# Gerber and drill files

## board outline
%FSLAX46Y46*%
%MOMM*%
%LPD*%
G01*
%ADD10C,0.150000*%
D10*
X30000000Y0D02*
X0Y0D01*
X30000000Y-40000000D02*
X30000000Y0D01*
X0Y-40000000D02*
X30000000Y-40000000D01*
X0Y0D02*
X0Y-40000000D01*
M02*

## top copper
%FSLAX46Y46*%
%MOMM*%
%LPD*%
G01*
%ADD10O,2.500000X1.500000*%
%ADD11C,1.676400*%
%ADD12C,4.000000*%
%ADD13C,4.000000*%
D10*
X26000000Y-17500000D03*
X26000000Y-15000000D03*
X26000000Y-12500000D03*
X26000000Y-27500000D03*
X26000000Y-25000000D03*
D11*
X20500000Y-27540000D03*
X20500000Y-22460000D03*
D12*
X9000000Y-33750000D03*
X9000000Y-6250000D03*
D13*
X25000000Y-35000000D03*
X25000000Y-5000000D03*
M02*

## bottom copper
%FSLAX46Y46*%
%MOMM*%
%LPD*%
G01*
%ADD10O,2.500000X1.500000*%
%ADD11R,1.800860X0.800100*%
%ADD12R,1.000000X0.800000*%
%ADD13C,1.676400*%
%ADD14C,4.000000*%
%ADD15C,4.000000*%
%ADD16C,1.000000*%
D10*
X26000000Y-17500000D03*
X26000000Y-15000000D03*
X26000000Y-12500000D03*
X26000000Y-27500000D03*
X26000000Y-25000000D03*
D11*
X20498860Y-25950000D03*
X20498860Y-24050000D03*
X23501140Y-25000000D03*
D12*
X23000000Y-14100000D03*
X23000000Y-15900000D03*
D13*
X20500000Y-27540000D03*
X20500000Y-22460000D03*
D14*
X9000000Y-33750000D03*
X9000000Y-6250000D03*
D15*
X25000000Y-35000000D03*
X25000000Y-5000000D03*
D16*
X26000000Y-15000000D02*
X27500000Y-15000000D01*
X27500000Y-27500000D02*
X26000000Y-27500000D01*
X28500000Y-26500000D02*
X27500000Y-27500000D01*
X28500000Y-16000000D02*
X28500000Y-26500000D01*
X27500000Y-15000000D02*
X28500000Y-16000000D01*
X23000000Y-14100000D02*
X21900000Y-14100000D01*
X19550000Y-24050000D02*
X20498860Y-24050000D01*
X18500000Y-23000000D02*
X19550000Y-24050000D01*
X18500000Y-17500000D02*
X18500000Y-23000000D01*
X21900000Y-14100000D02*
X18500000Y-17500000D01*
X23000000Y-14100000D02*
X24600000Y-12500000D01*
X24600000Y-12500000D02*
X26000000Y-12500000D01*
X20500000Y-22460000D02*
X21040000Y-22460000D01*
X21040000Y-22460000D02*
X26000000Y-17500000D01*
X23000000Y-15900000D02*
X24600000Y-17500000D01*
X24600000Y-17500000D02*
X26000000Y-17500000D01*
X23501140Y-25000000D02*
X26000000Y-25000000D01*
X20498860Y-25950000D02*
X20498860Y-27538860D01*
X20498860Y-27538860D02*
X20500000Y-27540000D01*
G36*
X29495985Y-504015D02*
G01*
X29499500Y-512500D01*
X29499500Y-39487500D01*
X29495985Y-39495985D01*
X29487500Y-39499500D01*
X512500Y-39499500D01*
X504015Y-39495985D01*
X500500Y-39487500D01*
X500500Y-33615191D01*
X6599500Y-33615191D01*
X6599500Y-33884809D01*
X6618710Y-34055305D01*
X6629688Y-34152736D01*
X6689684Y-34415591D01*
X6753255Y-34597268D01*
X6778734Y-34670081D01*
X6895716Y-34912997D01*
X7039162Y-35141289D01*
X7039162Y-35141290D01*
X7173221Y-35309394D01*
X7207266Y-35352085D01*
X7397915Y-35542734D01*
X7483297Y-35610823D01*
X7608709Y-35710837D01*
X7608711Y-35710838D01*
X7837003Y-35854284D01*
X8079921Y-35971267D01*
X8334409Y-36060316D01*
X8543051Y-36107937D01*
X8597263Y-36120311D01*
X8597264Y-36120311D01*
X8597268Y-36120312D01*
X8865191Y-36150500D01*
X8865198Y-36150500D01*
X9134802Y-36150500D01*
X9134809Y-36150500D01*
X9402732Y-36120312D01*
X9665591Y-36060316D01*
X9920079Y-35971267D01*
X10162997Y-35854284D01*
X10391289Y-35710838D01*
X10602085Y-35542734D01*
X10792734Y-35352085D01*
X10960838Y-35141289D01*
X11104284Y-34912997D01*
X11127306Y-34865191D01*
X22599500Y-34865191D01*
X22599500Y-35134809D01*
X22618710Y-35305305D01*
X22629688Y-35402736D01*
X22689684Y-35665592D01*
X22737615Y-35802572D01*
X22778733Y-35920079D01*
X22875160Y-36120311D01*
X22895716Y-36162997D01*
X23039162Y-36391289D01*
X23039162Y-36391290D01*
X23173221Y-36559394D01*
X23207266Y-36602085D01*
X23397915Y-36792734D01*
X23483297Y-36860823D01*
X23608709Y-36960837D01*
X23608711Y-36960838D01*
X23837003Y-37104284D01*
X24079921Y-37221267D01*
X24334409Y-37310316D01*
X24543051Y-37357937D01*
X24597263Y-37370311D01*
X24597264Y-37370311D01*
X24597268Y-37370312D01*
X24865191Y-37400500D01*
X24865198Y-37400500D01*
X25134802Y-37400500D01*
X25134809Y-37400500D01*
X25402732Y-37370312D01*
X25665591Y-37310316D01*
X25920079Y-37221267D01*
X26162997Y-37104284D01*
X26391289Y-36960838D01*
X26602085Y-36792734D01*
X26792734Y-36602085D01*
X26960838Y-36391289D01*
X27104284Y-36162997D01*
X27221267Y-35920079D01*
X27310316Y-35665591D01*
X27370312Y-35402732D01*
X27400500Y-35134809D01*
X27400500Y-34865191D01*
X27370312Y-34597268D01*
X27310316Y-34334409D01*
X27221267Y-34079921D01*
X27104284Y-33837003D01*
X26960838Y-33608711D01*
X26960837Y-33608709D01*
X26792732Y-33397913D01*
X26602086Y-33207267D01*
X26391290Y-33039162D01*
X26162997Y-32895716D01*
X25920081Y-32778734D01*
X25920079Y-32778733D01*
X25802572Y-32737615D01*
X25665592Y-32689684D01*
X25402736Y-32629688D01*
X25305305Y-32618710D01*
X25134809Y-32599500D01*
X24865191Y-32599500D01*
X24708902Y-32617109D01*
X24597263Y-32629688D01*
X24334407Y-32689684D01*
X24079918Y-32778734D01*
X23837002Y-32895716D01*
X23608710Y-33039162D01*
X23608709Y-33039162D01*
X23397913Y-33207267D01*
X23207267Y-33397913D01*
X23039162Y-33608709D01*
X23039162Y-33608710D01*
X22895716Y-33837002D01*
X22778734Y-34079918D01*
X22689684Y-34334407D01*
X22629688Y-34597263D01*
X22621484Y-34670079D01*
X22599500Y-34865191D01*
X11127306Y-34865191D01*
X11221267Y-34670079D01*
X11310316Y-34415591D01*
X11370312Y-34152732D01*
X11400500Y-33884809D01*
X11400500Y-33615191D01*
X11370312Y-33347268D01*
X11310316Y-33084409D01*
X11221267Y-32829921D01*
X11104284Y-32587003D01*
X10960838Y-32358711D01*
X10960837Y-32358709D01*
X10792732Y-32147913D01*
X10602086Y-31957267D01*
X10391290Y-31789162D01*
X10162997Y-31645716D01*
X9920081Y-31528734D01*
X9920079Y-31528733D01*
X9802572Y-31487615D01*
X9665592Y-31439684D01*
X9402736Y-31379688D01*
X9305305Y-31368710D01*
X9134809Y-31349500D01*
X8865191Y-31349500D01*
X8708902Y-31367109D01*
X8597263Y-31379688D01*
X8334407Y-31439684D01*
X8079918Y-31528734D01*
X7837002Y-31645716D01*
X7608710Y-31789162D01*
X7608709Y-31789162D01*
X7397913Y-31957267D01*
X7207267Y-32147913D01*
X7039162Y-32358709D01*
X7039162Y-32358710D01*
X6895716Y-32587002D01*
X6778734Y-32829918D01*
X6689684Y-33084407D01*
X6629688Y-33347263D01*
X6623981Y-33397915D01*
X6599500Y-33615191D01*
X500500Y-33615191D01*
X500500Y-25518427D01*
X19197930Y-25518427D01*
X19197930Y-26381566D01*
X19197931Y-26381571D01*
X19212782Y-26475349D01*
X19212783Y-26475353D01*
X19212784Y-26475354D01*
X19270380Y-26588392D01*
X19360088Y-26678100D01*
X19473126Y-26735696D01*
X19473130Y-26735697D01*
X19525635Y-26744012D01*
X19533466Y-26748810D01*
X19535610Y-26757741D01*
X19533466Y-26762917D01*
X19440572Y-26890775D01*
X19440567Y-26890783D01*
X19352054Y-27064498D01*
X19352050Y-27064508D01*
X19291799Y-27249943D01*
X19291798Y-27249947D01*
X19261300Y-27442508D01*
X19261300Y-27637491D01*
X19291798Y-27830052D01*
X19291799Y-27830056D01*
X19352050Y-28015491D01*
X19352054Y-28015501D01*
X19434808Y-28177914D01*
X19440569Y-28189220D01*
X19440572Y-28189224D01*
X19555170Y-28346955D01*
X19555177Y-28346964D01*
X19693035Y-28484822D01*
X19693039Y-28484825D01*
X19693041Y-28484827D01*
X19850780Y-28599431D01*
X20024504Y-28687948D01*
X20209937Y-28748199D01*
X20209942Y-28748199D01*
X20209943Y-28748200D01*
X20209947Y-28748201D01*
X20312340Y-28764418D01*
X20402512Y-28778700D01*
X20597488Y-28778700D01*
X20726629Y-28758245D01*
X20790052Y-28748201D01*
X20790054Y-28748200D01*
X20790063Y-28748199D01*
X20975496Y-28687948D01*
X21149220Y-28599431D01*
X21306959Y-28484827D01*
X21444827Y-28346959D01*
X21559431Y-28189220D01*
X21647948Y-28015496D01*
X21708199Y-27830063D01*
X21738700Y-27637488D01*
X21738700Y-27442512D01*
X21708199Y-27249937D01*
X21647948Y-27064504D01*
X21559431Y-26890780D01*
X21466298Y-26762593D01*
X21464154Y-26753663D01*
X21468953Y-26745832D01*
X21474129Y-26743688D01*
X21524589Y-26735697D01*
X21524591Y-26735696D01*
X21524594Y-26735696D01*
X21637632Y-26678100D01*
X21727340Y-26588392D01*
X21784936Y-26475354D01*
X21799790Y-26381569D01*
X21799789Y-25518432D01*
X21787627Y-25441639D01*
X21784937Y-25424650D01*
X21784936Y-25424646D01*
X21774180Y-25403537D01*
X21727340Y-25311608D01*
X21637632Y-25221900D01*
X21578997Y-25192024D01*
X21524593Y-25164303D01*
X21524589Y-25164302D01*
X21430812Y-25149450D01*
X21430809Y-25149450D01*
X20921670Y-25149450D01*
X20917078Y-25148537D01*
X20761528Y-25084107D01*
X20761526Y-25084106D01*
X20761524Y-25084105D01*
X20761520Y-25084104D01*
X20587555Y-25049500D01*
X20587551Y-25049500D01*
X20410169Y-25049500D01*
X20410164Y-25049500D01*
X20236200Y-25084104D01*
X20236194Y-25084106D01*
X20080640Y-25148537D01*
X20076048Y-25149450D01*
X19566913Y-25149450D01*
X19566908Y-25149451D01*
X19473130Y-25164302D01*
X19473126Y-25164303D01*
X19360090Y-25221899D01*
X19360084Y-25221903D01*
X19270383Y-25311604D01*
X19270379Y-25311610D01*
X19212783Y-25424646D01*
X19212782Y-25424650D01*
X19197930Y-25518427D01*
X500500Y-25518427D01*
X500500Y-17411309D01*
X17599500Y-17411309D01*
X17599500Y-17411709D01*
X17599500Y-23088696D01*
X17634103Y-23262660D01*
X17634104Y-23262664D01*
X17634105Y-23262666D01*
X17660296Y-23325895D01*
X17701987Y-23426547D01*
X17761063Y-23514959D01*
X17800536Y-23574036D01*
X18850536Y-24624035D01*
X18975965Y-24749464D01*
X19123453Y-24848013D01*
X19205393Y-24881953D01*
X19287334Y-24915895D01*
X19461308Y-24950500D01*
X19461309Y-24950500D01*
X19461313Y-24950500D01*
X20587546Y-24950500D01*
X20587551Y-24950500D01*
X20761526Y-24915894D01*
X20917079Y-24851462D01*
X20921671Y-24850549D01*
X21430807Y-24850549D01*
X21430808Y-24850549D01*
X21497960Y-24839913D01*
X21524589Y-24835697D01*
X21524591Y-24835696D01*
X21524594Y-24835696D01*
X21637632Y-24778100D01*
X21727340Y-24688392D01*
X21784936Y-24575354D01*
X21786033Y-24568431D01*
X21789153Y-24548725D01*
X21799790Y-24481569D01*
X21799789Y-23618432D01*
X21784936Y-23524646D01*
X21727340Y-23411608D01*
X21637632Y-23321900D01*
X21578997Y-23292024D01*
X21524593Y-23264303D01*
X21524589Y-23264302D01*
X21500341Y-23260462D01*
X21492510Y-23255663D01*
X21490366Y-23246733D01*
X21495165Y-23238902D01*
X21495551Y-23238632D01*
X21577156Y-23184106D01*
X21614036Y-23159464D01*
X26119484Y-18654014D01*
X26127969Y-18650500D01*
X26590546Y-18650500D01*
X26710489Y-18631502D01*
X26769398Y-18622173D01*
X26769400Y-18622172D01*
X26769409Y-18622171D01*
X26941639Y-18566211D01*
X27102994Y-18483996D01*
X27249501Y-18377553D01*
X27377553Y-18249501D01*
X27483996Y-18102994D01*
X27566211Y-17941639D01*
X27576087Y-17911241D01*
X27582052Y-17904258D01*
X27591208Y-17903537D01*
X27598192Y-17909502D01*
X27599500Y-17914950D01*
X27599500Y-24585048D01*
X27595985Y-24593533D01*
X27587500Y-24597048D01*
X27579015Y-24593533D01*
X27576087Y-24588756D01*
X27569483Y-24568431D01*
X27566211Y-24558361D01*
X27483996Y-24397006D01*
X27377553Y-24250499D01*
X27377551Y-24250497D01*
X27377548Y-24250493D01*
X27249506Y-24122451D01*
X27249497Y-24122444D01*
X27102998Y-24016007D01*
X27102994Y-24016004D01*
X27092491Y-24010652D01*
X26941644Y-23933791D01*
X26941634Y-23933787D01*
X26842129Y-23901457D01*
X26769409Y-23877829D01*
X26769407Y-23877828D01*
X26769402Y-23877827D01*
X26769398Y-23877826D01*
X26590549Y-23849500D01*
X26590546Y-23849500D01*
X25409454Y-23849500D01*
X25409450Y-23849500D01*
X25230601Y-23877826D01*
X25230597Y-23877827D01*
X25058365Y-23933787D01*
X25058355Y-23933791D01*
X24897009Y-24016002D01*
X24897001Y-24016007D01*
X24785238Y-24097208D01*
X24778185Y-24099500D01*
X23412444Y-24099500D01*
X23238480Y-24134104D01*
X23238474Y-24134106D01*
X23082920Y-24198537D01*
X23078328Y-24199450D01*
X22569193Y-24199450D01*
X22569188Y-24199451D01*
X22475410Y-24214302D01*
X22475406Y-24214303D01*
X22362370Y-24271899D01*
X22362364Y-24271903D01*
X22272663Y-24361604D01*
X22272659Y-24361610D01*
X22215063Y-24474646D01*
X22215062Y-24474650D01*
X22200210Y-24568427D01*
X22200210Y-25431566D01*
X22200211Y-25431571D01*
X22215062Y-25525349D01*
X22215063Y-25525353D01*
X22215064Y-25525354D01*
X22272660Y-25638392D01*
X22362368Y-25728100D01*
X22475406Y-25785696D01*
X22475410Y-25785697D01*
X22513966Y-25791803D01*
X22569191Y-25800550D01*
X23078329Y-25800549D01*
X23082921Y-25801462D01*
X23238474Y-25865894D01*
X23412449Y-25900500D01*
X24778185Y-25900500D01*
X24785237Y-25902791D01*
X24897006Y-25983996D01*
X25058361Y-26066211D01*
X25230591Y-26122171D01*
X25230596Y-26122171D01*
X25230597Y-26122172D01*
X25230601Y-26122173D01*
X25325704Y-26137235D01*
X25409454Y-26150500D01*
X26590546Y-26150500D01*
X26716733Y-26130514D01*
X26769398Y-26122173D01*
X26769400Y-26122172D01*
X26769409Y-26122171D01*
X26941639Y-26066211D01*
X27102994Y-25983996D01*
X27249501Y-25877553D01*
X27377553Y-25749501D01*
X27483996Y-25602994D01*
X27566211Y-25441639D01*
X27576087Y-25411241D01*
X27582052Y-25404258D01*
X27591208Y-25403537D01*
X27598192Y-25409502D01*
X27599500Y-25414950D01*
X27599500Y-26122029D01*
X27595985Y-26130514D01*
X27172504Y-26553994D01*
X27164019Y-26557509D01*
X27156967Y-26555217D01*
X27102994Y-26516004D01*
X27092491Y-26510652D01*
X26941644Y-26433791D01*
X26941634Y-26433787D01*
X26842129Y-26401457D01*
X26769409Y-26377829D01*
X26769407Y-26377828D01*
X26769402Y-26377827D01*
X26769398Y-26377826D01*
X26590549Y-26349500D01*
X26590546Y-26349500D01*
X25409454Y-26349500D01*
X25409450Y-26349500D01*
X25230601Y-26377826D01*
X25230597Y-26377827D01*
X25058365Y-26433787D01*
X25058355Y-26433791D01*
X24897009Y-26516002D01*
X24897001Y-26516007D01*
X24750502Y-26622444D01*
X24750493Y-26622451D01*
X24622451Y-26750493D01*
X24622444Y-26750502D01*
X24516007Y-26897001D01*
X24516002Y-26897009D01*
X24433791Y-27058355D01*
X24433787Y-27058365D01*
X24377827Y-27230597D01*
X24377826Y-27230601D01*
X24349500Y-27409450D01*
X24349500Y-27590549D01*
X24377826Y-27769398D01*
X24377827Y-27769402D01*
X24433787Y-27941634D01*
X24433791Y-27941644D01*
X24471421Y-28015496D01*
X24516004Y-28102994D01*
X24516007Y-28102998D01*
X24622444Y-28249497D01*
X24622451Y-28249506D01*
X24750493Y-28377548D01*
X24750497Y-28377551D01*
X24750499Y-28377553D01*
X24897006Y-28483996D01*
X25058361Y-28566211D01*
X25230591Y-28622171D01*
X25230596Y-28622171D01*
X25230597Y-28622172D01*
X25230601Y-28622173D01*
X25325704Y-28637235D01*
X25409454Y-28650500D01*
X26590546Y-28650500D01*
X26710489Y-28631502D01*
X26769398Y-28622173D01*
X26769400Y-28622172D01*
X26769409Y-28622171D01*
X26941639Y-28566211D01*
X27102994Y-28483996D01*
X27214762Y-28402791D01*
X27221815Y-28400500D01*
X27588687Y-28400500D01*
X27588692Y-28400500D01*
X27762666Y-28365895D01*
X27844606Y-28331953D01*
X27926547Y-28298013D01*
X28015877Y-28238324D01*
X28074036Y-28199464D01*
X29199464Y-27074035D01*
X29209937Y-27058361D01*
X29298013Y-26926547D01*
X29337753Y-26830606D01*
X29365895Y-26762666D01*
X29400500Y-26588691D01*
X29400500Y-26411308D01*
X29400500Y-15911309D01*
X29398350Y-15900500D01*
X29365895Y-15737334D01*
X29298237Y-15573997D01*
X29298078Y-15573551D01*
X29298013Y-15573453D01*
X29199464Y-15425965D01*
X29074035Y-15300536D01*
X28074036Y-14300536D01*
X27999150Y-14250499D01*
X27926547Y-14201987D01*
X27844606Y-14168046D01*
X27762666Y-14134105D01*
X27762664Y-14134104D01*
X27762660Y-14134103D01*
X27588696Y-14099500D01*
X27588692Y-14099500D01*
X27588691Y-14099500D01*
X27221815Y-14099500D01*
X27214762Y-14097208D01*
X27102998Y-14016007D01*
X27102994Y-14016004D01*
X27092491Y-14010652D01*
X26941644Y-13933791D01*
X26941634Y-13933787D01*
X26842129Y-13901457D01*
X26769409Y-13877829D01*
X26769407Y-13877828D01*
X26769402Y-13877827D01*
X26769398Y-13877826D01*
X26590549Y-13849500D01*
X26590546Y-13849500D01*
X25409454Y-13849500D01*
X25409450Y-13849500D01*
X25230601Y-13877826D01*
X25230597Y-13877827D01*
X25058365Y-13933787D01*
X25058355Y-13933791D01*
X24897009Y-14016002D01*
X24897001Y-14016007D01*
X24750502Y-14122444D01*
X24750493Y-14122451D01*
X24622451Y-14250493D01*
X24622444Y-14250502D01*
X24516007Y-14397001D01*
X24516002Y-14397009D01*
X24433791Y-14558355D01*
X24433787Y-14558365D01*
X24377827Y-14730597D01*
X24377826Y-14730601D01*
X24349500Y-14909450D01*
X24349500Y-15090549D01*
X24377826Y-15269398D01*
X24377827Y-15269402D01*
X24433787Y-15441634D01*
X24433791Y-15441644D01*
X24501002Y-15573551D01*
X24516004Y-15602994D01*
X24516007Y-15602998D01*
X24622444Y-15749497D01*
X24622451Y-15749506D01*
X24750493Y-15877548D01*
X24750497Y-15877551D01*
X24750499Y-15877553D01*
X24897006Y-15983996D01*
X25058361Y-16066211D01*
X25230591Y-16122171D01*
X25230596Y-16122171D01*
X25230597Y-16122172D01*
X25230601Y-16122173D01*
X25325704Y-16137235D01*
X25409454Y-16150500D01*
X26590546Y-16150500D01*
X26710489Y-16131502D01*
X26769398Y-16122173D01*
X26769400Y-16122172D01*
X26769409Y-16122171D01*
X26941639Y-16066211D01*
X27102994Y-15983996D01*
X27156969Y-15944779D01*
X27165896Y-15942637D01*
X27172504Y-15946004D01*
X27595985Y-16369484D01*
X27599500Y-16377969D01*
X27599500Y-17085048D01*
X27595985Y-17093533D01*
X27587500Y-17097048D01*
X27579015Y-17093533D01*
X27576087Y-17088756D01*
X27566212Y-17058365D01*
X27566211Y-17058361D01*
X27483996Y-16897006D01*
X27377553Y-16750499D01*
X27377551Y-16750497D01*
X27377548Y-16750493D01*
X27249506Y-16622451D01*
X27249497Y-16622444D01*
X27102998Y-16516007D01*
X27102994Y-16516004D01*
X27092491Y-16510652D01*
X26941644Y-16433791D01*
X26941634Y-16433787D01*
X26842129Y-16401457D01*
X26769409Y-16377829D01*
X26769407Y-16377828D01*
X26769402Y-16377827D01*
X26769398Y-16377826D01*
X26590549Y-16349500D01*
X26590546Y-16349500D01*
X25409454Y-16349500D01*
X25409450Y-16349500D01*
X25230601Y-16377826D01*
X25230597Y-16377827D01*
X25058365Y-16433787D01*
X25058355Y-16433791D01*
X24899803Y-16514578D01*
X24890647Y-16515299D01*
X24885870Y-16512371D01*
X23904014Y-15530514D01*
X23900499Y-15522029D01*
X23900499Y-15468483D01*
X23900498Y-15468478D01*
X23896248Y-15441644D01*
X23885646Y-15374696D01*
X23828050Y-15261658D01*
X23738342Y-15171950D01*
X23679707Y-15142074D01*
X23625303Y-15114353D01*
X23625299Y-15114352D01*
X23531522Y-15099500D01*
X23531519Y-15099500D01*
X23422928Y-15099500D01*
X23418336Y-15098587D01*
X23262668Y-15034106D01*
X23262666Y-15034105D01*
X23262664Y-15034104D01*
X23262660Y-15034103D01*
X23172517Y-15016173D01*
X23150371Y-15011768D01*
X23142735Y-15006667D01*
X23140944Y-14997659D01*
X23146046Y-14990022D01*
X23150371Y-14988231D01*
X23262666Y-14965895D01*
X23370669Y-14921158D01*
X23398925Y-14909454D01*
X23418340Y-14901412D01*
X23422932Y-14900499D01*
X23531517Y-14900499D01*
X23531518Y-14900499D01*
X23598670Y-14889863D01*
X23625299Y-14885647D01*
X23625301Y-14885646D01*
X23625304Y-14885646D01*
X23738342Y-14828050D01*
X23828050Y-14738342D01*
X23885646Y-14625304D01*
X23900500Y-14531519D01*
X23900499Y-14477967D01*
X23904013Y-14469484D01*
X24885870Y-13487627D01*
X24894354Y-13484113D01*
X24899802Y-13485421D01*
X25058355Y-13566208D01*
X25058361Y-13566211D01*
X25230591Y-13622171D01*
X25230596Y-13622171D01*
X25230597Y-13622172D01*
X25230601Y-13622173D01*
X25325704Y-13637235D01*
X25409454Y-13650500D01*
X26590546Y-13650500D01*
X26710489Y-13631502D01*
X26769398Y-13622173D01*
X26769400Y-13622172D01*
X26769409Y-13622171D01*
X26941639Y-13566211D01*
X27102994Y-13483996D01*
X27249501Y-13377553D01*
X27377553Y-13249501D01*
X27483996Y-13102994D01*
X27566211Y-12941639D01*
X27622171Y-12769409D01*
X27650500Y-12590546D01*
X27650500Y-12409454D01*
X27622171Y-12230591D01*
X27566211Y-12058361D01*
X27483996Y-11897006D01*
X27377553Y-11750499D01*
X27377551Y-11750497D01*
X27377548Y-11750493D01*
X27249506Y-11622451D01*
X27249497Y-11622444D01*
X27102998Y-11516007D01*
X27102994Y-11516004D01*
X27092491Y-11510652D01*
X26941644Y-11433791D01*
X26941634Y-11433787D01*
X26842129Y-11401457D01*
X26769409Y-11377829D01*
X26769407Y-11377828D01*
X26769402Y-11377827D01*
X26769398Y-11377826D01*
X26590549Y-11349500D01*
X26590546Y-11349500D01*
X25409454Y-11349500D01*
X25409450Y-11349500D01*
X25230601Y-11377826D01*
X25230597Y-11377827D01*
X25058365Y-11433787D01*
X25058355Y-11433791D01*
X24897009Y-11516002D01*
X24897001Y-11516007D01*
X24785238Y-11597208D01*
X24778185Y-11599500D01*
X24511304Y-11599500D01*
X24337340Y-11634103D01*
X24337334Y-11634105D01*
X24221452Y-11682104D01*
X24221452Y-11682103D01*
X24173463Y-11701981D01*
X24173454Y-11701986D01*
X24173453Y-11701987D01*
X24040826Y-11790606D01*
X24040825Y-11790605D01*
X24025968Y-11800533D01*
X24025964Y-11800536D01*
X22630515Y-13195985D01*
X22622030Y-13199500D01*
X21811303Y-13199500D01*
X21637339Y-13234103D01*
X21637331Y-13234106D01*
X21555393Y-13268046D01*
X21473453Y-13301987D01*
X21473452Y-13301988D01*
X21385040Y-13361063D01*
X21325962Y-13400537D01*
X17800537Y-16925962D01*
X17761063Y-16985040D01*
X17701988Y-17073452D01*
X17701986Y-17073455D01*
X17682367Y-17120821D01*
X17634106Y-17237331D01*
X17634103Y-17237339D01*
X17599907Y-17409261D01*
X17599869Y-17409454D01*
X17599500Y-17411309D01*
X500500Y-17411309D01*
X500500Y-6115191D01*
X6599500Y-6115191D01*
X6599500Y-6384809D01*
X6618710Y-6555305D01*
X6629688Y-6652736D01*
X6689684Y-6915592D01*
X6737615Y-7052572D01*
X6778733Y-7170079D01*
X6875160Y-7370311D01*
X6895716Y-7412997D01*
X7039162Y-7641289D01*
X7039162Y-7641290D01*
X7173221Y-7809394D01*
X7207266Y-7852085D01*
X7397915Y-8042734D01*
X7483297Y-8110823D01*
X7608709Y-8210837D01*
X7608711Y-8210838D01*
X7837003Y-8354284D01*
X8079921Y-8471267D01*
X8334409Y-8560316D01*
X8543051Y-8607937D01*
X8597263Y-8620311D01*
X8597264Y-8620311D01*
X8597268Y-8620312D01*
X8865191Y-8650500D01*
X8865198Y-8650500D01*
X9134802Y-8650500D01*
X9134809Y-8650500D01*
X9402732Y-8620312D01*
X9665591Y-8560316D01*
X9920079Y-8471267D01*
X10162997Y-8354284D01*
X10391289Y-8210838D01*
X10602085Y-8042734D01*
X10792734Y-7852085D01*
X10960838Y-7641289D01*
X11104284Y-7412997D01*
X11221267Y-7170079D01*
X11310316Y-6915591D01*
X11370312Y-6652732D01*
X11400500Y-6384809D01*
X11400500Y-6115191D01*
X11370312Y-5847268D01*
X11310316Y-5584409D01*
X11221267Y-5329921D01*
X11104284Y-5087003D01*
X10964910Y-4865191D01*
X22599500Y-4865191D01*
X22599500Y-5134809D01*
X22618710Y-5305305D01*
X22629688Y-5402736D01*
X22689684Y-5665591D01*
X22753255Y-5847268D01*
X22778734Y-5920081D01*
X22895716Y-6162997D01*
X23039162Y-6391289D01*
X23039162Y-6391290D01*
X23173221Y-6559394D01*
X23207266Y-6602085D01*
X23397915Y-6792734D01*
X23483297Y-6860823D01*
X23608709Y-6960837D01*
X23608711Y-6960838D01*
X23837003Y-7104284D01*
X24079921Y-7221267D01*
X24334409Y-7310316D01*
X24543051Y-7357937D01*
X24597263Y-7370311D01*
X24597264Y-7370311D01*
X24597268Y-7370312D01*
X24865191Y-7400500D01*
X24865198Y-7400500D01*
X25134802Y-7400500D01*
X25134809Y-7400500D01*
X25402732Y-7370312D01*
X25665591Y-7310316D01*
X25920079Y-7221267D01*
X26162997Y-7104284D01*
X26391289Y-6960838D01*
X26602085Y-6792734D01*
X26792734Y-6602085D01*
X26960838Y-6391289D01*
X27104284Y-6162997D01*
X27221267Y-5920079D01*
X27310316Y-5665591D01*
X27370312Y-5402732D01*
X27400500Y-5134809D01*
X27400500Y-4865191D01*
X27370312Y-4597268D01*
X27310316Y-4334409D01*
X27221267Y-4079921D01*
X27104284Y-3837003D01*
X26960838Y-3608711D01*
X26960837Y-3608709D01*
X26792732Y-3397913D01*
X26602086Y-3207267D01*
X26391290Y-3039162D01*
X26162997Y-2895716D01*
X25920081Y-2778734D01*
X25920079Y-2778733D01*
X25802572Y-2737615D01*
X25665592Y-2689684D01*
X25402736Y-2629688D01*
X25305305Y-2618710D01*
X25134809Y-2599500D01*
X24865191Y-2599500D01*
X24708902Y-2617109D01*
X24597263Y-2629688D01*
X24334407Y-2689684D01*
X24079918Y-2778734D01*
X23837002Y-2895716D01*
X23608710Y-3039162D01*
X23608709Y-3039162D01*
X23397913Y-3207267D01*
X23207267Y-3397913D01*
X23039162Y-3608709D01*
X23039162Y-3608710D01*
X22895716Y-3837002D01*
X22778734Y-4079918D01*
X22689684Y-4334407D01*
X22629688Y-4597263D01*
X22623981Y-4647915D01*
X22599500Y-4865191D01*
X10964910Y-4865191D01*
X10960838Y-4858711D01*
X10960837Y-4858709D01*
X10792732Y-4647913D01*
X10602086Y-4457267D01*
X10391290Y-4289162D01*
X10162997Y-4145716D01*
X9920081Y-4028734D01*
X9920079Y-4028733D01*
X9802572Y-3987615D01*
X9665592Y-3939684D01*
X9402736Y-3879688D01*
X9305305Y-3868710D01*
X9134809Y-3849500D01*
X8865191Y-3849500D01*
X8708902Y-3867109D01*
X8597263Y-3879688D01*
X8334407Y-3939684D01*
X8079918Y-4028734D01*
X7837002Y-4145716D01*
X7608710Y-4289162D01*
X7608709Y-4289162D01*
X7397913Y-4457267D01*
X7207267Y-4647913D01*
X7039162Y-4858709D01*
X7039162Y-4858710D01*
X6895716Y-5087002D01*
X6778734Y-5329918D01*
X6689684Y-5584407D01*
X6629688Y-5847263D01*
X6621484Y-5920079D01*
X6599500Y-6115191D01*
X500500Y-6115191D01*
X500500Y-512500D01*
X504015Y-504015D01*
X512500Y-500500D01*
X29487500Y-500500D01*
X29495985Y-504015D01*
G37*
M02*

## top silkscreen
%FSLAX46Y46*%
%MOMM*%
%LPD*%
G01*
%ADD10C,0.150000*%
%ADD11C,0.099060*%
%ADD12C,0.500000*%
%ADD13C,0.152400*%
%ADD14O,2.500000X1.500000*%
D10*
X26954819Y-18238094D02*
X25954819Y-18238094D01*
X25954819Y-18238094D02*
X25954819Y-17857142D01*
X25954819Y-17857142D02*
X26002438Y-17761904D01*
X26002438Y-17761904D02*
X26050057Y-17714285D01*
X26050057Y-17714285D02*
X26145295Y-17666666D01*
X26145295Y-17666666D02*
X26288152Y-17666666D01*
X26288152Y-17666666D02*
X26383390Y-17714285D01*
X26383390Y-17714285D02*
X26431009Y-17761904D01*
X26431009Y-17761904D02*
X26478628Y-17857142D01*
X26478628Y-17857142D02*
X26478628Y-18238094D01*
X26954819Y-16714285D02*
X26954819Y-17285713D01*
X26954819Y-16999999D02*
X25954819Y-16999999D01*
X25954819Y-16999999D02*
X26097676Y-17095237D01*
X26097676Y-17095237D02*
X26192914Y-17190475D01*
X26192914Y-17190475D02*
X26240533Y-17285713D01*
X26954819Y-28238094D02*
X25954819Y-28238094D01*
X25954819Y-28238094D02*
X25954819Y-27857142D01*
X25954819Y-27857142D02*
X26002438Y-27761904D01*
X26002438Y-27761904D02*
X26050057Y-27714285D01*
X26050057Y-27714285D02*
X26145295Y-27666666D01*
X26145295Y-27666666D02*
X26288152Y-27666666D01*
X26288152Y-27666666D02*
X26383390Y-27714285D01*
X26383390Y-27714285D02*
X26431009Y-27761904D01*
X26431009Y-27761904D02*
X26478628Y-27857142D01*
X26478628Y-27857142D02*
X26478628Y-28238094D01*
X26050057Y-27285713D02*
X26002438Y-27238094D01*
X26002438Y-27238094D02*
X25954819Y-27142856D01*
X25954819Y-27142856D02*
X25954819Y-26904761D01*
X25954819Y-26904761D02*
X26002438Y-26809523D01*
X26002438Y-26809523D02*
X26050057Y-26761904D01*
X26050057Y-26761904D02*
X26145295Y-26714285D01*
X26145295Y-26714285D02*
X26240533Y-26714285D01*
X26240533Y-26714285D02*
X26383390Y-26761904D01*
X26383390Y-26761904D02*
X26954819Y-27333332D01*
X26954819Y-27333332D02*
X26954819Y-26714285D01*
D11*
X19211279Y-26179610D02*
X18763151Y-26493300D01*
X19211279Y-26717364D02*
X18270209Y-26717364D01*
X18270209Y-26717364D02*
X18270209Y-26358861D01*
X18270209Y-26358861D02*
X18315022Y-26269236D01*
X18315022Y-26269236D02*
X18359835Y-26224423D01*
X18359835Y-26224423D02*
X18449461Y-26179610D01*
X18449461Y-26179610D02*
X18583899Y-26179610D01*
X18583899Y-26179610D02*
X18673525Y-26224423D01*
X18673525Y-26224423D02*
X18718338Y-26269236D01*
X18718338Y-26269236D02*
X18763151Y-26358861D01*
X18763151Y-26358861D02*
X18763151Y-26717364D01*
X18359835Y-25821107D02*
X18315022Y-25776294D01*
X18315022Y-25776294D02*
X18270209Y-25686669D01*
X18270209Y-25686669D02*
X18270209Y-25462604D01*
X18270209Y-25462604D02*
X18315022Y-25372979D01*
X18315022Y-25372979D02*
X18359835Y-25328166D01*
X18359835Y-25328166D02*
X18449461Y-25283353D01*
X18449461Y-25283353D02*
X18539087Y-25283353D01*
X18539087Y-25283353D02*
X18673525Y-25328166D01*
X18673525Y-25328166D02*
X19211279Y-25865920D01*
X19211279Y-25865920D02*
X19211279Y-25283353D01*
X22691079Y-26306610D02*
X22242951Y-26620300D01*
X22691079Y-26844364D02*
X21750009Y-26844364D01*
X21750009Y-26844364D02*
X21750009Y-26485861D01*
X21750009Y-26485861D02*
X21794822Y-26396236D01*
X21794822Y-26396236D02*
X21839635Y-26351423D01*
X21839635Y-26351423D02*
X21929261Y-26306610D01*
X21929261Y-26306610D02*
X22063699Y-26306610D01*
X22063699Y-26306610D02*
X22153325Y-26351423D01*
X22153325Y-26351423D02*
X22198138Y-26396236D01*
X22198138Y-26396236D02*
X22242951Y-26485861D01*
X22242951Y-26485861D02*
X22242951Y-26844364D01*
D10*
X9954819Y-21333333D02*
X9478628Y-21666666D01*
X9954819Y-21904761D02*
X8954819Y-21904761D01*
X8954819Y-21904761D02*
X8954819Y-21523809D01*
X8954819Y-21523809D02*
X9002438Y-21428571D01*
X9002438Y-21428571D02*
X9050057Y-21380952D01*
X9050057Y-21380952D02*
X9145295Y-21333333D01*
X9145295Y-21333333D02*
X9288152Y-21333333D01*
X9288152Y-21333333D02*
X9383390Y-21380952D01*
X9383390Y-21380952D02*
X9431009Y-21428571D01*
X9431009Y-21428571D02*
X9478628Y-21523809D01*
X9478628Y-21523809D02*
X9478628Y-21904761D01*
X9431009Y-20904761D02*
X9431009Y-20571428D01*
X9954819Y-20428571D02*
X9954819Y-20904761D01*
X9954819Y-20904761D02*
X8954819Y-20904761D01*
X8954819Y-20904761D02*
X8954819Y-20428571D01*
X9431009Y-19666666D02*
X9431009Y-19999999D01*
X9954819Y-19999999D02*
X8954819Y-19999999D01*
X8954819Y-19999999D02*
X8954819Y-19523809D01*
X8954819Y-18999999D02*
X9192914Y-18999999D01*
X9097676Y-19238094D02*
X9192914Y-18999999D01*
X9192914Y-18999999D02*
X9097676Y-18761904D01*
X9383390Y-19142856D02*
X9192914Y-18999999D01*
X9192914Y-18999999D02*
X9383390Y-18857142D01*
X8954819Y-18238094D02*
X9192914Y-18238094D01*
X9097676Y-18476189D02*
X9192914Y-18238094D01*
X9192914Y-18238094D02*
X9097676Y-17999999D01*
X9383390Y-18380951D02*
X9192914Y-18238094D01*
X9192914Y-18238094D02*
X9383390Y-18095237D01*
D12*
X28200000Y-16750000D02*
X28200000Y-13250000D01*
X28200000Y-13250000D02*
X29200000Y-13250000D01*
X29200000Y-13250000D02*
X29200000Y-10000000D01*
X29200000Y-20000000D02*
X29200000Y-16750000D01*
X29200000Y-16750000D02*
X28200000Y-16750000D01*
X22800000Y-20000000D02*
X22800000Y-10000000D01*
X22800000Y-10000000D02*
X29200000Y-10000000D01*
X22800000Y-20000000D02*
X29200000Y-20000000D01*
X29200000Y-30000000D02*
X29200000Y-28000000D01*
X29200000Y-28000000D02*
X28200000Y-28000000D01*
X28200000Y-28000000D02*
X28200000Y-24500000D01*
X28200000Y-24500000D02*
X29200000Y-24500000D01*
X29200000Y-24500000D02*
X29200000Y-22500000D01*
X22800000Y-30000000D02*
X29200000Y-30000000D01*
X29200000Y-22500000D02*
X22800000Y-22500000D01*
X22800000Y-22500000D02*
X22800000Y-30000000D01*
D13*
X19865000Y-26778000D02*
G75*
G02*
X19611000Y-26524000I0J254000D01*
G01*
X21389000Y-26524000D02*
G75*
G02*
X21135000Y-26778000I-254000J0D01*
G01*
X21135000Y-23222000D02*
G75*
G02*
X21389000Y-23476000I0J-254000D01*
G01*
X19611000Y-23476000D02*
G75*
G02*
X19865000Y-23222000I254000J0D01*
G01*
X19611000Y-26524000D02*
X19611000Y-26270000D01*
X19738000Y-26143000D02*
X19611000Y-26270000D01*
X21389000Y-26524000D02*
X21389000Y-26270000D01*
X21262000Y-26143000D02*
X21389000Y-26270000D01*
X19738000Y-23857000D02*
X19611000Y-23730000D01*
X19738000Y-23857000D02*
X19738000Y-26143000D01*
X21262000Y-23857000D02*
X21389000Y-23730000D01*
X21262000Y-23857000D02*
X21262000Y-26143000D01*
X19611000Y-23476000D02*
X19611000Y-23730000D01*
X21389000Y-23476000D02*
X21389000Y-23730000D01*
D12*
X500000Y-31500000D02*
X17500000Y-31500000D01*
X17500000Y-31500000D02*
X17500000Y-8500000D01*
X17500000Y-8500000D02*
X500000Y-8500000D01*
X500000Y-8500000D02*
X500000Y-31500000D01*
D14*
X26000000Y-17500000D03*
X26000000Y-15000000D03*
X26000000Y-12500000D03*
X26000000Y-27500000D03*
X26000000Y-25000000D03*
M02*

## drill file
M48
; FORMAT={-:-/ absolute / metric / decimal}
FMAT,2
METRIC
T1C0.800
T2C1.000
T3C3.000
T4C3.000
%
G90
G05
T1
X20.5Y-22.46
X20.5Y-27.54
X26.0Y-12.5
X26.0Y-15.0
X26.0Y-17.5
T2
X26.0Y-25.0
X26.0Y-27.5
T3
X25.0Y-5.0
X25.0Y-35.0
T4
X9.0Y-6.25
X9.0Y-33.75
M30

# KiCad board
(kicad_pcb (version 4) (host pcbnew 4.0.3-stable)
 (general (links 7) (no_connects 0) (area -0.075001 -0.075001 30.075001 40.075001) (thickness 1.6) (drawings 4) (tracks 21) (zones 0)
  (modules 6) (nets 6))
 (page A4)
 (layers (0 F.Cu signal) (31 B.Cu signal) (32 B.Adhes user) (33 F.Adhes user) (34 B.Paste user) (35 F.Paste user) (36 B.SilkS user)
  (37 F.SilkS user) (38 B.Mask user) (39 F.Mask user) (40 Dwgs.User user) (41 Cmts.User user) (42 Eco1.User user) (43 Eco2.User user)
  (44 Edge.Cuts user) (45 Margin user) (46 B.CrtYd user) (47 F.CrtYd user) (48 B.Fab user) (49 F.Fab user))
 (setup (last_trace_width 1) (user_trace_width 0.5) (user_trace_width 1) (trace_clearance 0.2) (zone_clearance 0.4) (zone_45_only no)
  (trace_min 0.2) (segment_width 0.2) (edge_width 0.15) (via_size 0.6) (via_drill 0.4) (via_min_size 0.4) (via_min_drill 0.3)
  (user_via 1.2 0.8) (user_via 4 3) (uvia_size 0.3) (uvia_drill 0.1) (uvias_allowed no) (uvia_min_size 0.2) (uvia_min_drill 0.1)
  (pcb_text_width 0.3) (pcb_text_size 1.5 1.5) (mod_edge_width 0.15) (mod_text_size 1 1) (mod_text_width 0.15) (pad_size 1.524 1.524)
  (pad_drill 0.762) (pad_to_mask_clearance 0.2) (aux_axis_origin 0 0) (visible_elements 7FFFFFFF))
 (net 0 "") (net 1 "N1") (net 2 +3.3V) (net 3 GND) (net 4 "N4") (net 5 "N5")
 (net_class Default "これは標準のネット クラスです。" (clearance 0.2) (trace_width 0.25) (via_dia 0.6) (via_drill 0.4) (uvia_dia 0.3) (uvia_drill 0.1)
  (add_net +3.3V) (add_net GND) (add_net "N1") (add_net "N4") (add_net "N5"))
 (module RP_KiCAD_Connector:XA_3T (layer F.Cu) (at 26 17.5 90)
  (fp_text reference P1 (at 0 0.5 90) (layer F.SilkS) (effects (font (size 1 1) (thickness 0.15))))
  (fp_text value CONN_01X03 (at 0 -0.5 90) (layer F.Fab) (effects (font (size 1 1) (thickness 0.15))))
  (fp_line (start 0.75 2.2) (end 4.25 2.2) (layer F.SilkS) (width 0.5))
  (fp_line (start 4.25 2.2) (end 4.25 3.2) (layer F.SilkS) (width 0.5))
  (fp_line (start 4.25 3.2) (end 7.5 3.2) (layer F.SilkS) (width 0.5))
  (fp_line (start -2.5 3.2) (end 0.75 3.2) (layer F.SilkS) (width 0.5))
  (fp_line (start 0.75 3.2) (end 0.75 2.2) (layer F.SilkS) (width 0.5))
  (fp_line (start -2.5 -3.2) (end 7.5 -3.2) (layer F.SilkS) (width 0.5))
  (fp_line (start 7.5 -3.2) (end 7.5 3.2) (layer F.SilkS) (width 0.5))
  (fp_line (start -2.5 -3.2) (end -2.5 3.2) (layer F.SilkS) (width 0.5))
  (pad 3 thru_hole oval (at 0 0 90) (size 1.5 2.5) (drill 0.8) (layers *.Cu *.Mask F.SilkS) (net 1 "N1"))
  (pad 2 thru_hole oval (at 2.5 0 90) (size 1.5 2.5) (drill 0.8) (layers *.Cu *.Mask F.SilkS) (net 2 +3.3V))
  (pad 1 thru_hole oval (at 5 0 90) (size 1.5 2.5) (drill 0.8) (layers *.Cu *.Mask F.SilkS) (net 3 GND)))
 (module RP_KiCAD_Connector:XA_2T (layer F.Cu) (at 26 27.5 90)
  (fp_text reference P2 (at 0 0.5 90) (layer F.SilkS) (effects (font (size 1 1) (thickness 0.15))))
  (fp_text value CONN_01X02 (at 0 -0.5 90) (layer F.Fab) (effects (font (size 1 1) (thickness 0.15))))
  (fp_line (start -2.5 3.2) (end -0.5 3.2) (layer F.SilkS) (width 0.5))
  (fp_line (start -0.5 3.2) (end -0.5 2.2) (layer F.SilkS) (width 0.5))
  (fp_line (start -0.5 2.2) (end 3 2.2) (layer F.SilkS) (width 0.5))
  (fp_line (start 3 2.2) (end 3 3.2) (layer F.SilkS) (width 0.5))
  (fp_line (start 3 3.2) (end 5 3.2) (layer F.SilkS) (width 0.5))
  (fp_line (start -2.5 -3.2) (end -2.5 3.2) (layer F.SilkS) (width 0.5))
  (fp_line (start 5 3.2) (end 5 -3.2) (layer F.SilkS) (width 0.5))
  (fp_line (start 5 -3.2) (end -2.5 -3.2) (layer F.SilkS) (width 0.5))
  (pad 2 thru_hole oval (at 0 0 90) (size 1.5 2.5) (drill 1) (layers *.Cu *.Mask F.SilkS) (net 2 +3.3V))
  (pad 1 thru_hole oval (at 2.5 0 90) (size 1.5 2.5) (drill 1) (layers *.Cu *.Mask F.SilkS) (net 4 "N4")))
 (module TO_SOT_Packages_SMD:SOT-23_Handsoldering (layer B.Cu) (at 22 25 90)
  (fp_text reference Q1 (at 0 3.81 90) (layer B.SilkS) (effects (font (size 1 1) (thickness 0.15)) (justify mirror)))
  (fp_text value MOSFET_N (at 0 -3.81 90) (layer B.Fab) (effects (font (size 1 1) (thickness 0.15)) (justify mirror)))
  (pad G smd rect (at -0.95 -1.50114 90) (size 0.8001 1.80086) (layers B.Cu B.Paste B.Mask) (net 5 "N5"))
  (pad S smd rect (at 0.95 -1.50114 90) (size 0.8001 1.80086) (layers B.Cu B.Paste B.Mask) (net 3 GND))
  (pad D smd rect (at 0 1.50114 90) (size 0.8001 1.80086) (layers B.Cu B.Paste B.Mask) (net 4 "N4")))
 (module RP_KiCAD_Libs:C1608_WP (layer B.Cu) (at 23 15 270)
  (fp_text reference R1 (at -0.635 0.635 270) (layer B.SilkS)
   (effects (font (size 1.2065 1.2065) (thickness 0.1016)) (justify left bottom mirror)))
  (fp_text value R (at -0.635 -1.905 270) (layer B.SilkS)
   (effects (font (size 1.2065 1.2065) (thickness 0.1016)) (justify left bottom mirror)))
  (pad 1 smd rect (at -0.9 0 270) (size 0.8 1) (layers B.Cu B.Paste B.Mask) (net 3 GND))
  (pad 2 smd rect (at 0.9 0 270) (size 0.8 1) (layers B.Cu B.Paste B.Mask) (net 1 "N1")))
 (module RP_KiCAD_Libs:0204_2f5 (layer F.Cu) (at 20.5 25 90)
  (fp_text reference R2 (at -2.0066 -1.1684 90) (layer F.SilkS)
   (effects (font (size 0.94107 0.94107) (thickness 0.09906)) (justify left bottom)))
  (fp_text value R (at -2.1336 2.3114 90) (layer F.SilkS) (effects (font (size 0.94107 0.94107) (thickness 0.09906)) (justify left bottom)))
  (fp_arc (start -1.524 -0.635) (end -1.778 -0.635) (angle 90) (layer F.SilkS) (width 0.1524))
  (fp_arc (start -1.524 0.635) (end -1.778 0.635) (angle -90) (layer F.SilkS) (width 0.1524))
  (fp_arc (start 1.524 0.635) (end 1.524 0.889) (angle -90) (layer F.SilkS) (width 0.1524))
  (fp_arc (start 1.524 -0.635) (end 1.524 -0.889) (angle 90) (layer F.SilkS) (width 0.1524))
  (fp_line (start -1.524 -0.889) (end -1.27 -0.889) (layer F.SilkS) (width 0.1524))
  (fp_line (start -1.143 -0.762) (end -1.27 -0.889) (layer F.SilkS) (width 0.1524))
  (fp_line (start -1.524 0.889) (end -1.27 0.889) (layer F.SilkS) (width 0.1524))
  (fp_line (start -1.143 0.762) (end -1.27 0.889) (layer F.SilkS) (width 0.1524))
  (fp_line (start 1.143 -0.762) (end 1.27 -0.889) (layer F.SilkS) (width 0.1524))
  (fp_line (start 1.143 -0.762) (end -1.143 -0.762) (layer F.SilkS) (width 0.1524))
  (fp_line (start 1.143 0.762) (end 1.27 0.889) (layer F.SilkS) (width 0.1524))
  (fp_line (start 1.143 0.762) (end -1.143 0.762) (layer F.SilkS) (width 0.1524))
  (fp_line (start 1.524 -0.889) (end 1.27 -0.889) (layer F.SilkS) (width 0.1524))
  (fp_line (start 1.524 0.889) (end 1.27 0.889) (layer F.SilkS) (width 0.1524))
  (pad 1 thru_hole circle (at -2.54 0 90) (size 1.6764 1.6764) (drill 0.8) (layers *.Cu *.Mask) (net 5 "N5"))
  (pad 2 thru_hole circle (at 2.54 0 90) (size 1.6764 1.6764) (drill 0.8) (layers *.Cu *.Mask) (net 1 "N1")))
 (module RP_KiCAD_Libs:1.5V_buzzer (layer F.Cu) (at 9 20 90)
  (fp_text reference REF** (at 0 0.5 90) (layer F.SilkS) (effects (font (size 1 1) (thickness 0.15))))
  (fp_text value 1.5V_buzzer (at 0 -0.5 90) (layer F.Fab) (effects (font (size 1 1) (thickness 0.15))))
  (fp_line (start -11.5 -8.5) (end -11.5 8.5) (layer F.SilkS) (width 0.5))
  (fp_line (start -11.5 8.5) (end 11.5 8.5) (layer F.SilkS) (width 0.5))
  (fp_line (start 11.5 8.5) (end 11.5 -8.5) (layer F.SilkS) (width 0.5))
  (fp_line (start 11.5 -8.5) (end -11.5 -8.5) (layer F.SilkS) (width 0.5))
  (pad 1 thru_hole circle (at -13.75 0 90) (size 4 4) (drill 3) (layers *.Cu *.Mask))
  (pad 2 thru_hole circle (at 13.75 0 90) (size 4 4) (drill 3) (layers *.Cu *.Mask)))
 (gr_line (start 30 0) (end 0 0) (angle 90) (layer Edge.Cuts) (width 0.15))
 (gr_line (start 30 40) (end 30 0) (angle 90) (layer Edge.Cuts) (width 0.15))
 (gr_line (start 0 40) (end 30 40) (angle 90) (layer Edge.Cuts) (width 0.15))
 (gr_line (start 0 0) (end 0 40) (angle 90) (layer Edge.Cuts) (width 0.15))
 (via (at 25 35) (size 4) (drill 3) (layers F.Cu B.Cu) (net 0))
 (via (at 25 5) (size 4) (drill 3) (layers F.Cu B.Cu) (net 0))
 (segment (start 26 15) (end 27.5 15) (width 1) (layer B.Cu) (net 2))
 (segment (start 27.5 27.5) (end 26 27.5) (width 1) (layer B.Cu) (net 2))
 (segment (start 28.5 26.5) (end 27.5 27.5) (width 1) (layer B.Cu) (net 2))
 (segment (start 28.5 16) (end 28.5 26.5) (width 1) (layer B.Cu) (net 2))
 (segment (start 27.5 15) (end 28.5 16) (width 1) (layer B.Cu) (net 2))
 (segment (start 23 14.1) (end 21.9 14.1) (width 1) (layer B.Cu) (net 3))
 (segment (start 19.55 24.05) (end 20.49886 24.05) (width 1) (layer B.Cu) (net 3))
 (segment (start 18.5 23) (end 19.55 24.05) (width 1) (layer B.Cu) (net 3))
 (segment (start 18.5 17.5) (end 18.5 23) (width 1) (layer B.Cu) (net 3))
 (segment (start 21.9 14.1) (end 18.5 17.5) (width 1) (layer B.Cu) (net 3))
 (segment (start 23 14.1) (end 24.6 12.5) (width 1) (layer B.Cu) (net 3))
 (segment (start 24.6 12.5) (end 26 12.5) (width 1) (layer B.Cu) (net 3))
 (segment (start 20.5 22.46) (end 21.04 22.46) (width 1) (layer B.Cu) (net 1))
 (segment (start 21.04 22.46) (end 26 17.5) (width 1) (layer B.Cu) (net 1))
 (segment (start 23 15.9) (end 24.6 17.5) (width 1) (layer B.Cu) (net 1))
 (segment (start 24.6 17.5) (end 26 17.5) (width 1) (layer B.Cu) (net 1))
 (segment (start 23.50114 25) (end 26 25) (width 1) (layer B.Cu) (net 4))
 (segment (start 20.49886 25.95) (end 20.49886 27.53886) (width 1) (layer B.Cu) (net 5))
 (segment (start 20.49886 27.53886) (end 20.5 27.54) (width 1) (layer B.Cu) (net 5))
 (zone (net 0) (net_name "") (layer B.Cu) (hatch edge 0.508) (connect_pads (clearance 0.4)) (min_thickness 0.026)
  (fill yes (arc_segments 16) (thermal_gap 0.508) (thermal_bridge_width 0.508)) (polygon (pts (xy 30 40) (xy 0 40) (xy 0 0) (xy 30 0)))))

